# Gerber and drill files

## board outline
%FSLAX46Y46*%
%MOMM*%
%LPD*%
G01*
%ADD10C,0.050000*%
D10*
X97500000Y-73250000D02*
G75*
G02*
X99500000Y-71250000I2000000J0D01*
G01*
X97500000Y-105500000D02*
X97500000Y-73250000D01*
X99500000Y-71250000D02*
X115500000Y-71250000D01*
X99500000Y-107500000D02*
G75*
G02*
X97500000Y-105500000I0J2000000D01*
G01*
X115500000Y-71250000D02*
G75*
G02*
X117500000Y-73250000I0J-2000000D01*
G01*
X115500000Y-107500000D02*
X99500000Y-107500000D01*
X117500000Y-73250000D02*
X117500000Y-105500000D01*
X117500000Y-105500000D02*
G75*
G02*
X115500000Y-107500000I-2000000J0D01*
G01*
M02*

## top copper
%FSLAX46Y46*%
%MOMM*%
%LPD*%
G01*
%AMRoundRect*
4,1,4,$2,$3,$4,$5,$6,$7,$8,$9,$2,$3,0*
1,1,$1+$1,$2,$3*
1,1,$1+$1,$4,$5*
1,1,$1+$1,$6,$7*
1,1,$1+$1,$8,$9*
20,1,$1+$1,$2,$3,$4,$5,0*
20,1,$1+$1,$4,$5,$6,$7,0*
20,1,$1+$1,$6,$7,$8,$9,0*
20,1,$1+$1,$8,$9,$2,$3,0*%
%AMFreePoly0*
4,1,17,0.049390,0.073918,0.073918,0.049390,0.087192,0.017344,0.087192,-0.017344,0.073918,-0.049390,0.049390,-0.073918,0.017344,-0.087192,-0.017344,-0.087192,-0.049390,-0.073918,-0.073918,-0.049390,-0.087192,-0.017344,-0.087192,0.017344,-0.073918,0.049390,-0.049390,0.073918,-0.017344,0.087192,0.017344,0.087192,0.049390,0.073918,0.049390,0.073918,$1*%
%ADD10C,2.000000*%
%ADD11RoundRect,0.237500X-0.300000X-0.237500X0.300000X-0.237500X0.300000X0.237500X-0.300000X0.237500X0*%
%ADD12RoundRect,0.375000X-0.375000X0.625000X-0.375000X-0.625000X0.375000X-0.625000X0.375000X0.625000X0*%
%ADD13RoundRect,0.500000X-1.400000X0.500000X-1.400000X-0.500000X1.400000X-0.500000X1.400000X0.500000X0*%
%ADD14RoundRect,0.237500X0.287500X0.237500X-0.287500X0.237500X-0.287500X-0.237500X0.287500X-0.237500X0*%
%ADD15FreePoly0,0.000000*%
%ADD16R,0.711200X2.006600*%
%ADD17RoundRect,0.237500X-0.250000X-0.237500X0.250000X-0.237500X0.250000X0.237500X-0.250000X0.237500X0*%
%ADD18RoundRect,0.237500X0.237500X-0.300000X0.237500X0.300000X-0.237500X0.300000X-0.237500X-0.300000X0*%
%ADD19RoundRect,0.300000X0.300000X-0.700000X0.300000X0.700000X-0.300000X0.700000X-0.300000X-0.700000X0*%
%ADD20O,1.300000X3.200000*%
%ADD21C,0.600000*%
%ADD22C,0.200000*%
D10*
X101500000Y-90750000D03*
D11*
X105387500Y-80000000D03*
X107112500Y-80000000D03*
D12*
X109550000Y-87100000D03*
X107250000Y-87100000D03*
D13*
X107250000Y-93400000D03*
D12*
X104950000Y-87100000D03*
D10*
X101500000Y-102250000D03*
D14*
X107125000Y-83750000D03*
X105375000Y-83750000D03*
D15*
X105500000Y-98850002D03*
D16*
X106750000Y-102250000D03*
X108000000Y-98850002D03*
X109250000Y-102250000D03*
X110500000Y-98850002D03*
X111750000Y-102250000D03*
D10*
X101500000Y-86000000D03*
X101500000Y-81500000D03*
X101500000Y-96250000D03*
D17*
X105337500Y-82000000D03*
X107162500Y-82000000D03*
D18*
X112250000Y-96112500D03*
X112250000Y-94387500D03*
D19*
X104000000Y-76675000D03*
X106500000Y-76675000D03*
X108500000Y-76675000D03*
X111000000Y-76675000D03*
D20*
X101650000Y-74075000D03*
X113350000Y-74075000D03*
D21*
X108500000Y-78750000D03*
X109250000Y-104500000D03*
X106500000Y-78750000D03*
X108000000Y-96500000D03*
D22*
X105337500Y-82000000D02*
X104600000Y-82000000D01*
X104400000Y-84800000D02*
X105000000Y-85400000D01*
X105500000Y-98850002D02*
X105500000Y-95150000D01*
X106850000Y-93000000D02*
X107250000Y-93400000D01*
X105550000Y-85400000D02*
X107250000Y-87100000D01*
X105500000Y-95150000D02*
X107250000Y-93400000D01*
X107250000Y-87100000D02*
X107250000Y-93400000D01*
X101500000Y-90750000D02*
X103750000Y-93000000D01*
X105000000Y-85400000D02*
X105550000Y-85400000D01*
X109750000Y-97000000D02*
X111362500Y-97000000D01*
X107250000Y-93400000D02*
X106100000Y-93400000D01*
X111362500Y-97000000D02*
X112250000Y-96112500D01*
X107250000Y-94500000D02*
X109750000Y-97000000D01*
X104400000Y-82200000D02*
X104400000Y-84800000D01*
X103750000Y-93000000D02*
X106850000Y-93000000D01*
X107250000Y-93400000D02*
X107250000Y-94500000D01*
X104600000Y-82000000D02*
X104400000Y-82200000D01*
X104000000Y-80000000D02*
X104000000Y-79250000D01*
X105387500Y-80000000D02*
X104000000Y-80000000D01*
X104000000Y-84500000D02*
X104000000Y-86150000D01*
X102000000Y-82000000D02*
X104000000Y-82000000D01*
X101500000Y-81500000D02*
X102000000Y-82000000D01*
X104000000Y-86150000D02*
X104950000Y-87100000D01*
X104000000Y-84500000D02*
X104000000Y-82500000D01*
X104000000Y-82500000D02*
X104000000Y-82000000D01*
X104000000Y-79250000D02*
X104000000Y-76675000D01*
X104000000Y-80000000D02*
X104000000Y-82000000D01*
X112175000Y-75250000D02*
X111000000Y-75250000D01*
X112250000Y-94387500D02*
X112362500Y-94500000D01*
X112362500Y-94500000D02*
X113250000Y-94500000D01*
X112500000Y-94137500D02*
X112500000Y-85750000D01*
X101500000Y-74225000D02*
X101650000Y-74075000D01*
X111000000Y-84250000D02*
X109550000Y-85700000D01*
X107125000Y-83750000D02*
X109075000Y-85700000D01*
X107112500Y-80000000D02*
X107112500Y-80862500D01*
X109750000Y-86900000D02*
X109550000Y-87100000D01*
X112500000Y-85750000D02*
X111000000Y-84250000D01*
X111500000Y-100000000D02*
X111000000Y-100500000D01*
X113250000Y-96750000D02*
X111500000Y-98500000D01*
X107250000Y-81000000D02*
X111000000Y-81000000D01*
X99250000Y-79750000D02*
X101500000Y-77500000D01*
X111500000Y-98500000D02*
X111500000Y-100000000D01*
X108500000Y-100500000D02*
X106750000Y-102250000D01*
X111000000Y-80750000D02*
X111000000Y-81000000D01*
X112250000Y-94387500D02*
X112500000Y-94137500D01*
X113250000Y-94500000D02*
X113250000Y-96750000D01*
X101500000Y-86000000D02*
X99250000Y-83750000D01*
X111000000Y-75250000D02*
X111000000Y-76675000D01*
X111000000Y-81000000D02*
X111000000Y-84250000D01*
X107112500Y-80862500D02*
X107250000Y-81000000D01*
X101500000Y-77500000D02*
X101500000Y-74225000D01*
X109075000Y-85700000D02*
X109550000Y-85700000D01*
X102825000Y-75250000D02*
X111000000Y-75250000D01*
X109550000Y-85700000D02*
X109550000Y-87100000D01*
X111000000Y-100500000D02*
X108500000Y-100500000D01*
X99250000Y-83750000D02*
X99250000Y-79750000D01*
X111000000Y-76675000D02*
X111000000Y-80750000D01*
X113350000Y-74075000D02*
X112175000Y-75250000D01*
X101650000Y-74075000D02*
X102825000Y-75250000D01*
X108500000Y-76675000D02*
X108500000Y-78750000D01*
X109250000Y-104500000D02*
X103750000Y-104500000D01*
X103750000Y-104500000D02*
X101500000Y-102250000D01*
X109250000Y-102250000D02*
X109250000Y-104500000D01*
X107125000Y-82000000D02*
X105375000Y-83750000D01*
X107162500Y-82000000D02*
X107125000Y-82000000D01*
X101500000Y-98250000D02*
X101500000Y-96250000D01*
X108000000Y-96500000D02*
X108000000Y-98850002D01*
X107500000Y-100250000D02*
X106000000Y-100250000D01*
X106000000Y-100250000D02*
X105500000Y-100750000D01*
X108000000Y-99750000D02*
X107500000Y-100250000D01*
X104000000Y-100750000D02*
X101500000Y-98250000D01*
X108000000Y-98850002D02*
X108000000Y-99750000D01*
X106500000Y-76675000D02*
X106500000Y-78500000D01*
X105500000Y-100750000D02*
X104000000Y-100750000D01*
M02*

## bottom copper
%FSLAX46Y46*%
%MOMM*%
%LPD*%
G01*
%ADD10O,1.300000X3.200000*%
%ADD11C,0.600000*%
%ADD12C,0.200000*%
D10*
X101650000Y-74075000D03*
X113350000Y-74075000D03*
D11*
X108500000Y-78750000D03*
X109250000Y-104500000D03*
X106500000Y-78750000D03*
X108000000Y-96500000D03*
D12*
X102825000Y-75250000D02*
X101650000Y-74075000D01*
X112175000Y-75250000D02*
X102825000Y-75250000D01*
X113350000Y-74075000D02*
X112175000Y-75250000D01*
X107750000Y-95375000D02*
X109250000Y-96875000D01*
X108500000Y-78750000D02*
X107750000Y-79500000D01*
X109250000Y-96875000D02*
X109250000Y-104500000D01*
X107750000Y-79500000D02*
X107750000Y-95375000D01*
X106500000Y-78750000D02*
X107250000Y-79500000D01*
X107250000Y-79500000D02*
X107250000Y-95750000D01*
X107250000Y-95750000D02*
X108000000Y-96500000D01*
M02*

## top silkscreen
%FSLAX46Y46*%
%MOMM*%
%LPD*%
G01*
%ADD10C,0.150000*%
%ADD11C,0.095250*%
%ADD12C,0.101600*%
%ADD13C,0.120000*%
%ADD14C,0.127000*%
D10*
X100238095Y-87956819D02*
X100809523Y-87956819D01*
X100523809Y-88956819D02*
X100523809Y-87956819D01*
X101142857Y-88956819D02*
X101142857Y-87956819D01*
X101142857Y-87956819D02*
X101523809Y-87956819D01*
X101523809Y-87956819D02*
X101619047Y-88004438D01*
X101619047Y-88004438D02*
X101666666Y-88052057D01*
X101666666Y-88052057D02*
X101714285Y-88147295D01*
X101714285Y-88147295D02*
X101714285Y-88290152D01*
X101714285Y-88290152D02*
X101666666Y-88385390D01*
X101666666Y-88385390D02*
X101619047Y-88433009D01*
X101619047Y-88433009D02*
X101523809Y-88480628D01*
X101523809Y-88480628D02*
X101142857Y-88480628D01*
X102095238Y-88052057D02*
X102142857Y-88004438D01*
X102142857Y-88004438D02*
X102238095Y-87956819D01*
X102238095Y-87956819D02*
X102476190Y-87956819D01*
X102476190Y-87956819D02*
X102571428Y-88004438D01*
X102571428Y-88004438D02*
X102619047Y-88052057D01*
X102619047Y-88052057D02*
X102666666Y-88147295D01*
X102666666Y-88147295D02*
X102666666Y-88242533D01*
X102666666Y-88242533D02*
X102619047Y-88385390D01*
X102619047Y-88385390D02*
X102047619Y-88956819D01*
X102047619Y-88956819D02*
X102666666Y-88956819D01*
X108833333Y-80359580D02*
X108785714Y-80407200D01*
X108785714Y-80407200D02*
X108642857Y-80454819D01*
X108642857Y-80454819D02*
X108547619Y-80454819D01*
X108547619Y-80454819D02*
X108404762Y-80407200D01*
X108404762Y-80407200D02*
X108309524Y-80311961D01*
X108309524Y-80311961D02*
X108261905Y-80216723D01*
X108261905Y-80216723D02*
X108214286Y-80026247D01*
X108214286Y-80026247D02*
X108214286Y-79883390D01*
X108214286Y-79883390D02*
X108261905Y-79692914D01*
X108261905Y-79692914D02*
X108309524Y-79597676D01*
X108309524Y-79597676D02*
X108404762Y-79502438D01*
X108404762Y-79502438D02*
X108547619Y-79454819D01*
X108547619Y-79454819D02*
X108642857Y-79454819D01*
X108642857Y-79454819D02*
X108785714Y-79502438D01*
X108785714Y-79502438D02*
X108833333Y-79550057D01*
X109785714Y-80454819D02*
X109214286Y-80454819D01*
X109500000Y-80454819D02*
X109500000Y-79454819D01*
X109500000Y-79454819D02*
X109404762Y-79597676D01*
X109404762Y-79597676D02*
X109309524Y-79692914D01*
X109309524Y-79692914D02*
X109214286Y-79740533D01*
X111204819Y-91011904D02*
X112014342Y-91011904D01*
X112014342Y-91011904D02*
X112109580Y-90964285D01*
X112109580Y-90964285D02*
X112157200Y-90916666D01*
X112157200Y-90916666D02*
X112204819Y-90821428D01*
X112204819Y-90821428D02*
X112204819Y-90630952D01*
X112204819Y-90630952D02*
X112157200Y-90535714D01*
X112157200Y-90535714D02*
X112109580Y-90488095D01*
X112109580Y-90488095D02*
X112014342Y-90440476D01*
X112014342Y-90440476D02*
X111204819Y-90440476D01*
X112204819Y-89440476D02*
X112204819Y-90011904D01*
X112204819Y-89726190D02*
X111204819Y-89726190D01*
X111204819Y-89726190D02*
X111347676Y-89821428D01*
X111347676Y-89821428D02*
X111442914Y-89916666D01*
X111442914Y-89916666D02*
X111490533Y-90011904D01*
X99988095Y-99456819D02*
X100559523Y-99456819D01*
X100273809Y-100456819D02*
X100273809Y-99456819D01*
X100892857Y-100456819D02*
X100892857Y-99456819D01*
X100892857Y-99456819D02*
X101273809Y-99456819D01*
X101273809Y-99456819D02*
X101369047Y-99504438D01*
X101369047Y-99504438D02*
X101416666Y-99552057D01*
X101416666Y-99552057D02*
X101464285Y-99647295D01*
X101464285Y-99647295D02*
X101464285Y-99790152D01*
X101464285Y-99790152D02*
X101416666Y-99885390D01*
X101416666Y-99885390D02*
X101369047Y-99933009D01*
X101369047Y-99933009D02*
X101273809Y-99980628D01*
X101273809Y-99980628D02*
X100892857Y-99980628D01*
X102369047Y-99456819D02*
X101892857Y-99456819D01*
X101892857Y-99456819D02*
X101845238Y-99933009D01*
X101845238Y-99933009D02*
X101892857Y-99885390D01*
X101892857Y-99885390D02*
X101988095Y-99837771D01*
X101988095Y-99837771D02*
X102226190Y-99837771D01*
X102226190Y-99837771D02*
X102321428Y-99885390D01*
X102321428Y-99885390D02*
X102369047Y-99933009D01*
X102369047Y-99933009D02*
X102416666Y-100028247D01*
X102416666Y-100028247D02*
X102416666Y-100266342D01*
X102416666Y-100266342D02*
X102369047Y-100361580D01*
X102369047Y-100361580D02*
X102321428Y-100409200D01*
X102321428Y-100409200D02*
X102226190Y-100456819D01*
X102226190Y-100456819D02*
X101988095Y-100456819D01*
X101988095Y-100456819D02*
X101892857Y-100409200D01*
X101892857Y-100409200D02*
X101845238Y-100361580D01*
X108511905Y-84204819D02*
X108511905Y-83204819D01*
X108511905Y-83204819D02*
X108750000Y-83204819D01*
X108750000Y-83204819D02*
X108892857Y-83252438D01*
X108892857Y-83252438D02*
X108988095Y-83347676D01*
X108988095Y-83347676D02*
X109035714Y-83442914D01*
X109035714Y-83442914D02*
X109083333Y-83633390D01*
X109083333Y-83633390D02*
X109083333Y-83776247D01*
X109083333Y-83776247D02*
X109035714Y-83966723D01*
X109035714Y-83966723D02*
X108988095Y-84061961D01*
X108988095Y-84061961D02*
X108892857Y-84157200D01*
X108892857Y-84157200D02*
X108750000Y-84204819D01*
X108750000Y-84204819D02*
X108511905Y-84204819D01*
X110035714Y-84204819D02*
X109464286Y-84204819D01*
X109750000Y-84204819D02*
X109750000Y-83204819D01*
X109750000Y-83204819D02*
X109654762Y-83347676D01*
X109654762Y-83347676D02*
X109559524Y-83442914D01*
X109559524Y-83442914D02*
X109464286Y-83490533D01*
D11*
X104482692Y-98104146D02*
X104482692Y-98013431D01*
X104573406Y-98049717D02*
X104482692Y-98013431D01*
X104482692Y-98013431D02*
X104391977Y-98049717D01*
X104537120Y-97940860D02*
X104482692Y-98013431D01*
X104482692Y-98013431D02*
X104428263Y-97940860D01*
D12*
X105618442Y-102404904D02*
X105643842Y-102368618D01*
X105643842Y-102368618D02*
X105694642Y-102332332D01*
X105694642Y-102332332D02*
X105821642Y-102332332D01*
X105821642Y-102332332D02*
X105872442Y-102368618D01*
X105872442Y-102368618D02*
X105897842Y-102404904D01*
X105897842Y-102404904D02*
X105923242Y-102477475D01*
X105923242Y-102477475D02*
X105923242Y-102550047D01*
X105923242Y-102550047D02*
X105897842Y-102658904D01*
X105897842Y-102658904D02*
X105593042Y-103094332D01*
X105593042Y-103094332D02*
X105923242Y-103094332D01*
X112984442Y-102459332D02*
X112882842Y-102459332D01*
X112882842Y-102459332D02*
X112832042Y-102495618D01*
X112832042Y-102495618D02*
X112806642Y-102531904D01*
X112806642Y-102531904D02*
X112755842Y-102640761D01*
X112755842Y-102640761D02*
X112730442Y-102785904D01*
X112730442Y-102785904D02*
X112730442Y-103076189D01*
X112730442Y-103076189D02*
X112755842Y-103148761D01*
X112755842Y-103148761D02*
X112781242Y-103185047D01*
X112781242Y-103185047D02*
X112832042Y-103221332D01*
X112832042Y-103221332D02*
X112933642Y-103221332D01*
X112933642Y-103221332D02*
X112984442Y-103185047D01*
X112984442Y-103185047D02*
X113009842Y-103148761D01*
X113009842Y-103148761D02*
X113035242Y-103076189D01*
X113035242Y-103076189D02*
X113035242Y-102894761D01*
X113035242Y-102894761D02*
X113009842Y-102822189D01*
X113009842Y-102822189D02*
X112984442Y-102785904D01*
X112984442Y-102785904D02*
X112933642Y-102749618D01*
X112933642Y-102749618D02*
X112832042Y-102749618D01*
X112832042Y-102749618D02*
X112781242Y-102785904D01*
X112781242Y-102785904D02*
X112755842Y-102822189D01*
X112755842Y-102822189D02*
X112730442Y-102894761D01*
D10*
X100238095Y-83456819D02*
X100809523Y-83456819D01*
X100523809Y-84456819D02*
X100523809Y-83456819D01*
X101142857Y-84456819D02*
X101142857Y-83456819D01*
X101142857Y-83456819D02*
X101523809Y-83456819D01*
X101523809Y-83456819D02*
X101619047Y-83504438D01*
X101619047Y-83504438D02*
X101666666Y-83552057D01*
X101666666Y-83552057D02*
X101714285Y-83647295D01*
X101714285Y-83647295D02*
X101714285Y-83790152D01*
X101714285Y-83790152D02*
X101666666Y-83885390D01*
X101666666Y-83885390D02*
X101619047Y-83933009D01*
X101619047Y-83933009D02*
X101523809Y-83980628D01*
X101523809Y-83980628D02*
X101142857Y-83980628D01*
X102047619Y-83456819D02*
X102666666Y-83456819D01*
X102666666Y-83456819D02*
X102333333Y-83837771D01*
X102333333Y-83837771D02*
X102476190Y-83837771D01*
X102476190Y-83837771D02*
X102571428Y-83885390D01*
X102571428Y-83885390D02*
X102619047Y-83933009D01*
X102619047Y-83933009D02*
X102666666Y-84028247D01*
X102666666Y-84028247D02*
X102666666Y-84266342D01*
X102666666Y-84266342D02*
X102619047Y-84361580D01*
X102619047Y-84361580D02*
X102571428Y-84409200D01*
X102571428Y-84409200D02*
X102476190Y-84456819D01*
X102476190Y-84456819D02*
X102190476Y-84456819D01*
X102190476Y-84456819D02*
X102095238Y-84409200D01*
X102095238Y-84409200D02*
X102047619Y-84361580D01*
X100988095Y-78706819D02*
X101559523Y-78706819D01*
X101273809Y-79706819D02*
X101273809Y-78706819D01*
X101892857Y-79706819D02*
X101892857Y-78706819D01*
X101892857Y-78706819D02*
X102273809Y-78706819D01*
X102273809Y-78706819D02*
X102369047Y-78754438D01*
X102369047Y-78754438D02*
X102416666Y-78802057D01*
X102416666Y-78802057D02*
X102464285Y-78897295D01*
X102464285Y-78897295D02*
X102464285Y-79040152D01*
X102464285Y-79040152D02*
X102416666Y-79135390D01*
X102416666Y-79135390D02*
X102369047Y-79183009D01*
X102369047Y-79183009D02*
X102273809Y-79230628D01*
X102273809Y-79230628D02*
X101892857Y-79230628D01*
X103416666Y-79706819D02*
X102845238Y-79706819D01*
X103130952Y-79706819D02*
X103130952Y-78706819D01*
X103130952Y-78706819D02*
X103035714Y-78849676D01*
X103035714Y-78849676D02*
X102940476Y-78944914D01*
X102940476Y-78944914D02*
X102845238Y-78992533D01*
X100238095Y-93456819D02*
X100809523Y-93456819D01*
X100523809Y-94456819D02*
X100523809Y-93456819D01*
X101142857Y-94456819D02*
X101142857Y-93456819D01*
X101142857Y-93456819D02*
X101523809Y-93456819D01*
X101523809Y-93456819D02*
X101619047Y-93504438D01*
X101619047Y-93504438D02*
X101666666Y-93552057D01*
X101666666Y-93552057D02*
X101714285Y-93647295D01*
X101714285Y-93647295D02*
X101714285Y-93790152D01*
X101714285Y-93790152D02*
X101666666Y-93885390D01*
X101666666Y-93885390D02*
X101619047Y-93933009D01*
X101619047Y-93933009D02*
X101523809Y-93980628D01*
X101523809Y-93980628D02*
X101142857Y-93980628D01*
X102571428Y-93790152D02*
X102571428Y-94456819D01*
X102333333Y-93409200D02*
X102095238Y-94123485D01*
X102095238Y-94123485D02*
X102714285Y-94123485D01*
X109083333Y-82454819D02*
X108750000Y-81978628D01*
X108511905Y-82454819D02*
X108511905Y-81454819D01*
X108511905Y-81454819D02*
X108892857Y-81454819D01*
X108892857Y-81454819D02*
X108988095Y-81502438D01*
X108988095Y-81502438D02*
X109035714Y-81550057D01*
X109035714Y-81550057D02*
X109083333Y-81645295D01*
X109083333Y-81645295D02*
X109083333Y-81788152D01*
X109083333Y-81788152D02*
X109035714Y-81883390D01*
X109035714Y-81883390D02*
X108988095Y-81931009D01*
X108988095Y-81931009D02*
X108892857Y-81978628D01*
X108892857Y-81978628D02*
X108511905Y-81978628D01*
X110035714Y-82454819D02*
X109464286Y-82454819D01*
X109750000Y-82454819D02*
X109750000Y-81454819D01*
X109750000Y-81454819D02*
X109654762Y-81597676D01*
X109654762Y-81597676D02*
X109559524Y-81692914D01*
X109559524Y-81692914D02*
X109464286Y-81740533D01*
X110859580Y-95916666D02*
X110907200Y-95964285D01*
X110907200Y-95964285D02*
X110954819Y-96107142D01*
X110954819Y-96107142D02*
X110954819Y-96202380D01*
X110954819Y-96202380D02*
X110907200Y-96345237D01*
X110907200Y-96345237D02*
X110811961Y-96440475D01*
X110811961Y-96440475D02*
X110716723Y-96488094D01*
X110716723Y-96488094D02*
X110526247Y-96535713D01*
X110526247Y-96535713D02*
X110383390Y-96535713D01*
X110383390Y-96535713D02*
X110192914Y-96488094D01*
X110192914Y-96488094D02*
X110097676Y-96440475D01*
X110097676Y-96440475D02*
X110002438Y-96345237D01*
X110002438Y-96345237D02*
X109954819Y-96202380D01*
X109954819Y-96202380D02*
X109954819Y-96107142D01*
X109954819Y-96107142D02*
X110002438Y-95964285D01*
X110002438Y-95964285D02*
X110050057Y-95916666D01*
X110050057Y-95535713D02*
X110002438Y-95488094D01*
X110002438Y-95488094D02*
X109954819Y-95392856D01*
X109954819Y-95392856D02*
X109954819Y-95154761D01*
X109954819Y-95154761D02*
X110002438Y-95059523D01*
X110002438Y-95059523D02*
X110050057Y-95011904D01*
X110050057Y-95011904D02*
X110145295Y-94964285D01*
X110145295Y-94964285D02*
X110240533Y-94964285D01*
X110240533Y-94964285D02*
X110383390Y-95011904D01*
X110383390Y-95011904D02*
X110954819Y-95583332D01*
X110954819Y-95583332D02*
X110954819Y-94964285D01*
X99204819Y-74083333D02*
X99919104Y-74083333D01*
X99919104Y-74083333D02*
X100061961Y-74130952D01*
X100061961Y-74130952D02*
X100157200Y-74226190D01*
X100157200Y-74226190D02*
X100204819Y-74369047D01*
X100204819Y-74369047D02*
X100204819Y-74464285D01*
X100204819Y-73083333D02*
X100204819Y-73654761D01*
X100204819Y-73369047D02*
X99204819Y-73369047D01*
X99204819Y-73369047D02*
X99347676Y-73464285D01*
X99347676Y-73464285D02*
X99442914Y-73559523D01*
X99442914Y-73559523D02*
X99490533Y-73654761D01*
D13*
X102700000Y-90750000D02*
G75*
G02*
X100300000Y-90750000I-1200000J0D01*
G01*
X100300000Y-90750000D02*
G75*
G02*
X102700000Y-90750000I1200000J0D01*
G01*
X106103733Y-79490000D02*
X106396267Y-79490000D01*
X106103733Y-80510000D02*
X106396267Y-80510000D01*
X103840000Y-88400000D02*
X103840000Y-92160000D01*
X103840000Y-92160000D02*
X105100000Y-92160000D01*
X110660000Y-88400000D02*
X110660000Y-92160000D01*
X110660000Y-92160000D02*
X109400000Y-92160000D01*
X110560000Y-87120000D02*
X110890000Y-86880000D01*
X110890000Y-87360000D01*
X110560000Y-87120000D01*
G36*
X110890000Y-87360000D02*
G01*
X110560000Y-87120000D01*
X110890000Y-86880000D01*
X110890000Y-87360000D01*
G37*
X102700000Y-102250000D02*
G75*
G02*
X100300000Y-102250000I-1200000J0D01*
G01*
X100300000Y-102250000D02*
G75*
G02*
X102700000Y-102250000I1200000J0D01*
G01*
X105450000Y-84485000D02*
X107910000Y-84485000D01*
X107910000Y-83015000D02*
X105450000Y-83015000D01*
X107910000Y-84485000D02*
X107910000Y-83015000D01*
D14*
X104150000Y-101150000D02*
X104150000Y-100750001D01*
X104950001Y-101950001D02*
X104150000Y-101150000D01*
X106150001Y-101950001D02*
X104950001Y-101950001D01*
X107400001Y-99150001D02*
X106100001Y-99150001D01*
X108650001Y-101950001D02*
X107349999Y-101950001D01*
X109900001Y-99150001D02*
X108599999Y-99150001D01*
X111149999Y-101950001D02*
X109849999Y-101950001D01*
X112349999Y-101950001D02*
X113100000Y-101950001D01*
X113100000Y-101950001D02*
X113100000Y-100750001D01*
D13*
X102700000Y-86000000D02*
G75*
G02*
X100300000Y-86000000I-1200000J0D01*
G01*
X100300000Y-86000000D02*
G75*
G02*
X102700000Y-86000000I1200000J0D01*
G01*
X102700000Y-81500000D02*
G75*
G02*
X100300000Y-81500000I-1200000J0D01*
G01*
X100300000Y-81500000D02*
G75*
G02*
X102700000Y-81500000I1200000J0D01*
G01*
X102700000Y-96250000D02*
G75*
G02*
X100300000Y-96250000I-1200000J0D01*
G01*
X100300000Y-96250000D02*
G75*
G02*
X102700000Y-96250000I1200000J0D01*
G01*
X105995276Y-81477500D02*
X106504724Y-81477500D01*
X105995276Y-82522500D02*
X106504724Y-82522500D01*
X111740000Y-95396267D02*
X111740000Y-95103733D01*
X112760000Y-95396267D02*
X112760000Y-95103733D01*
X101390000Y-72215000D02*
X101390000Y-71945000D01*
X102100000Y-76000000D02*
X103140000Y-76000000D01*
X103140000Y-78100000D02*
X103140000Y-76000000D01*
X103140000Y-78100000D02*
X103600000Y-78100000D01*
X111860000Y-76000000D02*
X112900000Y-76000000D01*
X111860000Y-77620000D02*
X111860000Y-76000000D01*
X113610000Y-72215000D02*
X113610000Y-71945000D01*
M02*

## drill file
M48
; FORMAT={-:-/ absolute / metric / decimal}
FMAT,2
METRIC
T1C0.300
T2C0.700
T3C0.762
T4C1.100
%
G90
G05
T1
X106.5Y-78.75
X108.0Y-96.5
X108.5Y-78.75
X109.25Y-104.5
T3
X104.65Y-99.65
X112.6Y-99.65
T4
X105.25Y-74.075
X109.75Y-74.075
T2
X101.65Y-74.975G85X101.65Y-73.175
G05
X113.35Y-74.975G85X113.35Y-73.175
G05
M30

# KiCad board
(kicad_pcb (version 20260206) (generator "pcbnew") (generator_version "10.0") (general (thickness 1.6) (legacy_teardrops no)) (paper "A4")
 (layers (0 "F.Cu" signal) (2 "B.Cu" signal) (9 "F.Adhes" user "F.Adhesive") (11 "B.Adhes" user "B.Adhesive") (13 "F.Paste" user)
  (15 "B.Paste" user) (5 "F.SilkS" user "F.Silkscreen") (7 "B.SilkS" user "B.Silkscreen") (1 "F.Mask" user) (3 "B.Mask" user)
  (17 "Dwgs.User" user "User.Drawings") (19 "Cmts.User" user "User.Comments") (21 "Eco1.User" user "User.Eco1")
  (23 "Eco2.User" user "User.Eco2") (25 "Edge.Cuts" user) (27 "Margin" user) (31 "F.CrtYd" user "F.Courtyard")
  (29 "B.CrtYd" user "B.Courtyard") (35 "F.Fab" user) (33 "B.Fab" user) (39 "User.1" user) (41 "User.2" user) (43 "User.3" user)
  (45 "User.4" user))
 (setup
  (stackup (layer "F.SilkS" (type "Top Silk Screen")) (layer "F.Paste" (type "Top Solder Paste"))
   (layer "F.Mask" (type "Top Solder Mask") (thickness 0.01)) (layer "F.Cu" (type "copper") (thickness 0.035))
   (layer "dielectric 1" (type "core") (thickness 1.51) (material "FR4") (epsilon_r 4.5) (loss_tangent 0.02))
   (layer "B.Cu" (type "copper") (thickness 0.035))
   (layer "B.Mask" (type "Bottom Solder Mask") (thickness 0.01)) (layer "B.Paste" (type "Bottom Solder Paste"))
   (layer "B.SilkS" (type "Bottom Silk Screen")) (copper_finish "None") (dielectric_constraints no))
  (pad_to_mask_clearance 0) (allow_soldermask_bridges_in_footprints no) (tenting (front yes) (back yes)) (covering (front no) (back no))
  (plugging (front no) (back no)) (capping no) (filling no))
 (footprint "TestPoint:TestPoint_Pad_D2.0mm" (layer "F.Cu") (at 101.5 90.75)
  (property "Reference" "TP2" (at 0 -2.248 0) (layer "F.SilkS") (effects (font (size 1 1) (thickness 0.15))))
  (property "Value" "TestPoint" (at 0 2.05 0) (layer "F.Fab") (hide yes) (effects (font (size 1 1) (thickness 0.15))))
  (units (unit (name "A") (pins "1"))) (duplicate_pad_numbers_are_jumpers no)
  (fp_circle (center 0 0) (end 0 1.2) (stroke (width 0.12) (type solid)) (fill no) (layer "F.SilkS"))
  (pad "1" smd circle (at 0 0) (size 2 2) (layers "F.Cu" "F.Mask") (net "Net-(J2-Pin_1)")))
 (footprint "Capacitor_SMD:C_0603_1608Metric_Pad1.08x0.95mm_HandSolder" (layer "F.Cu") (at 106.25 80)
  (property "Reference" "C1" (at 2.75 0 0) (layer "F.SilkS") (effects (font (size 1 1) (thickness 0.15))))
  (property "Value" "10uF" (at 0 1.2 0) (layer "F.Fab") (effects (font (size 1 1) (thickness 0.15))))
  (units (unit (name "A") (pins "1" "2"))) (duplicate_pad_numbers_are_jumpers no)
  (fp_line (start -0.146267 -0.51) (end 0.146267 -0.51) (stroke (width 0.12) (type solid)) (layer "F.SilkS"))
  (fp_line (start -0.146267 0.51) (end 0.146267 0.51) (stroke (width 0.12) (type solid)) (layer "F.SilkS"))
  (pad "1" smd roundrect (at -0.8625 0) (size 1.075 0.95) (layers "F.Cu" "F.Mask" "F.Paste") (roundrect_rratio 0.25) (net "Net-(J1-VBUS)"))
  (pad "2" smd roundrect (at 0.8625 0) (size 1.075 0.95) (layers "F.Cu" "F.Mask" "F.Paste") (roundrect_rratio 0.25) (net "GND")))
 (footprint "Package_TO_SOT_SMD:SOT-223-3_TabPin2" (layer "F.Cu") (at 107.25 90.25 -90)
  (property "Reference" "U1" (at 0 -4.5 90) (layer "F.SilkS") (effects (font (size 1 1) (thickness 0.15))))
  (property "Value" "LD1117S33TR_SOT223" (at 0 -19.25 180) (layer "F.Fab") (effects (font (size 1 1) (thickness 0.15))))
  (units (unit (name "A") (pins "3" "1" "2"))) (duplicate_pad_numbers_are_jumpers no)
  (fp_line (start -1.85 3.41) (end 1.91 3.41) (stroke (width 0.12) (type solid)) (layer "F.SilkS"))
  (fp_line (start 1.91 3.41) (end 1.91 2.15) (stroke (width 0.12) (type solid)) (layer "F.SilkS"))
  (fp_line (start -1.85 -3.41) (end 1.91 -3.41) (stroke (width 0.12) (type solid)) (layer "F.SilkS"))
  (fp_line (start 1.91 -3.41) (end 1.91 -2.15) (stroke (width 0.12) (type solid)) (layer "F.SilkS"))
  (fp_poly
   (pts (xy -3.13 -3.31) (xy -3.37 -3.64) (xy -2.89 -3.64) (xy -3.13 -3.31)) (stroke (width 0.12) (type solid)) (fill yes) (layer "F.SilkS"))
  (pad "1" smd roundrect (at -3.15 -2.3 270) (size 2 1.5) (layers "F.Cu" "F.Mask" "F.Paste") (roundrect_rratio 0.25) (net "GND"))
  (pad "2" smd roundrect (at -3.15 0 270) (size 2 1.5) (layers "F.Cu" "F.Mask" "F.Paste") (roundrect_rratio 0.25) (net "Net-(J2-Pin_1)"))
  (pad "2" smd roundrect (at 3.15 0 270) (size 2 3.8) (layers "F.Cu" "F.Mask" "F.Paste") (roundrect_rratio 0.25) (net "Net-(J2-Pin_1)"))
  (pad "3" smd roundrect (at -3.15 2.3 270) (size 2 1.5) (layers "F.Cu" "F.Mask" "F.Paste") (roundrect_rratio 0.25) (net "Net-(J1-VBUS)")))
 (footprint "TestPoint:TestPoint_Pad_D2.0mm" (layer "F.Cu") (at 101.5 102.25)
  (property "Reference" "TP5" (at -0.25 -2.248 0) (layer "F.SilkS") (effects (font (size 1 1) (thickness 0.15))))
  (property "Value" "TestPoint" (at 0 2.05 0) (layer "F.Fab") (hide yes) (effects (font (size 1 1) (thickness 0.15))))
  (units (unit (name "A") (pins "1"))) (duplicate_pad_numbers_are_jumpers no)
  (fp_circle (center 0 0) (end 0 1.2) (stroke (width 0.12) (type solid)) (fill no) (layer "F.SilkS"))
  (pad "1" smd circle (at 0 0) (size 2 2) (layers "F.Cu" "F.Mask") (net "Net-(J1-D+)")))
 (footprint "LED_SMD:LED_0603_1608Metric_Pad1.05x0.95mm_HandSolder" (layer "F.Cu") (at 106.25 83.75 180)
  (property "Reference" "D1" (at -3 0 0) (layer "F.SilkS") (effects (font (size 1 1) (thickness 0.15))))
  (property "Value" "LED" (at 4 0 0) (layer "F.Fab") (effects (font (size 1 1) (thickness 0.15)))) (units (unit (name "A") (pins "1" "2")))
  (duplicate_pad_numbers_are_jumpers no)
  (fp_line (start 0.8 -0.735) (end -1.66 -0.735) (stroke (width 0.12) (type solid)) (layer "F.SilkS"))
  (fp_line (start -1.66 0.735) (end 0.8 0.735) (stroke (width 0.12) (type solid)) (layer "F.SilkS"))
  (fp_line (start -1.66 -0.735) (end -1.66 0.735) (stroke (width 0.12) (type solid)) (layer "F.SilkS"))
  (pad "1" smd roundrect (at -0.875 0 180) (size 1.05 0.95) (layers "F.Cu" "F.Mask" "F.Paste") (roundrect_rratio 0.25) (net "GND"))
  (pad "2" smd roundrect (at 0.875 0 180) (size 1.05 0.95) (layers "F.Cu" "F.Mask" "F.Paste") (roundrect_rratio 0.25) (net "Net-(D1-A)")))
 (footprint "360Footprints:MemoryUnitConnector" (layer "F.Cu") (at 108.625 100.550001)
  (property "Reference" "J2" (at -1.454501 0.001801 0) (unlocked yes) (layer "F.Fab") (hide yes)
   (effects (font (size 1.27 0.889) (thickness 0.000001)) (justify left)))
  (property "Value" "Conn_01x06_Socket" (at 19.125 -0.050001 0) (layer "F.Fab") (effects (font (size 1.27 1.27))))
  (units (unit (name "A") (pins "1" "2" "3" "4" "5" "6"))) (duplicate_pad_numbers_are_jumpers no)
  (fp_line (start -4.475 0.599999) (end -4.475 0.2) (stroke (width 0.127) (type default)) (layer "F.SilkS"))
  (fp_line (start -3.674999 1.4) (end -4.475 0.599999) (stroke (width 0.127) (type default)) (layer "F.SilkS"))
  (fp_line (start -2.474999 1.4) (end -3.674999 1.4) (stroke (width 0.127) (type default)) (layer "F.SilkS"))
  (fp_line (start -1.224999 -1.4) (end -2.524999 -1.4) (stroke (width 0.127) (type default)) (layer "F.SilkS"))
  (fp_line (start 0.025001 1.4) (end -1.275001 1.4) (stroke (width 0.127) (type default)) (layer "F.SilkS"))
  (fp_line (start 1.275001 -1.4) (end -0.025001 -1.4) (stroke (width 0.127) (type default)) (layer "F.SilkS"))
  (fp_line (start 2.524999 1.4) (end 1.224999 1.4) (stroke (width 0.127) (type default)) (layer "F.SilkS"))
  (fp_line (start 3.724999 1.4) (end 4.475 1.4) (stroke (width 0.127) (type default)) (layer "F.SilkS"))
  (fp_line (start 4.475 1.4) (end 4.475 0.2) (stroke (width 0.127) (type default)) (layer "F.SilkS"))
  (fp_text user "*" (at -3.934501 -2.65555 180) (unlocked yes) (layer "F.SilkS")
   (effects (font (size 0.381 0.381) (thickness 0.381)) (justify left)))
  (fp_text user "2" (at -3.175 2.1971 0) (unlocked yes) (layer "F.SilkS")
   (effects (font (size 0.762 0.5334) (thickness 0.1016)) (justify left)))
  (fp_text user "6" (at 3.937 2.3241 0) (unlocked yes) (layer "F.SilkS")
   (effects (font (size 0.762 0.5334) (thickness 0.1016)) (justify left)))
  (pad "" np_thru_hole circle (at -3.975001 -0.900001) (size 0.508 0.508) (drill 0.762) (layers "*.Cu" "*.Mask"))
  (pad "" np_thru_hole circle (at 3.975001 -0.900001) (size 0.508 0.508) (drill 0.762) (layers "*.Cu" "*.Mask"))
  (pad "1" smd custom (at -3.125 -1.699999) (size 0.1778 0.1778) (layers "F.Cu" "F.Mask" "F.Paste") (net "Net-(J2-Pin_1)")
   (options (clearance outline) (anchor circle)) (primitives))
  (pad "2" smd rect (at -1.875 1.699999) (size 0.7112 2.0066) (layers "F.Cu" "F.Mask" "F.Paste") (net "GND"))
  (pad "3" smd rect (at -0.625 -1.699999) (size 0.7112 2.0066) (layers "F.Cu" "F.Mask" "F.Paste") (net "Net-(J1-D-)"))
  (pad "4" smd rect (at 0.625 1.699999) (size 0.7112 2.0066) (layers "F.Cu" "F.Mask" "F.Paste") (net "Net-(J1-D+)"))
  (pad "5" smd rect (at 1.875 -1.699999) (size 0.7112 2.0066) (layers "F.Cu" "F.Mask" "F.Paste") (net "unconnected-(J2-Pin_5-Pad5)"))
  (pad "6" smd rect (at 3.125 1.699999) (size 0.7112 2.0066) (layers "F.Cu" "F.Mask" "F.Paste") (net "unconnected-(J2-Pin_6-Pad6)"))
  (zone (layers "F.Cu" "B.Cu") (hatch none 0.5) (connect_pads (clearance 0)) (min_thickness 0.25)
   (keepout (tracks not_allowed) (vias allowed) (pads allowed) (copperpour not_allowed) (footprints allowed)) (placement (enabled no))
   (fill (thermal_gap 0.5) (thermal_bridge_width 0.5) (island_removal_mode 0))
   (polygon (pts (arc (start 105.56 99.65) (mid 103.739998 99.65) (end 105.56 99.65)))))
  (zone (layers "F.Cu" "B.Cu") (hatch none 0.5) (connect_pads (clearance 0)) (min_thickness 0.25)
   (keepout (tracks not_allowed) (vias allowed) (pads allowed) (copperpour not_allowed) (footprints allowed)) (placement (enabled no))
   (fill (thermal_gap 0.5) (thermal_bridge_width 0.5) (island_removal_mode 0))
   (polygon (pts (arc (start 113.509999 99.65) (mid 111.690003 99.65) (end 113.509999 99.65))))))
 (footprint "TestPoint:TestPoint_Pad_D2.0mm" (layer "F.Cu") (at 101.5 86)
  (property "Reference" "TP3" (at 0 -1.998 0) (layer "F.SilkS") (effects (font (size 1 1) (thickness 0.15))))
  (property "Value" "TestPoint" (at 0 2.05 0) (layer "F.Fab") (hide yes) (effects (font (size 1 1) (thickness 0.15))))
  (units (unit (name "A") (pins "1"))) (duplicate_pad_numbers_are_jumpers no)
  (fp_circle (center 0 0) (end 0 1.2) (stroke (width 0.12) (type solid)) (fill no) (layer "F.SilkS"))
  (pad "1" smd circle (at 0 0) (size 2 2) (layers "F.Cu" "F.Mask") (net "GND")))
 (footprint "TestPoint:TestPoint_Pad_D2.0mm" (layer "F.Cu") (at 101.5 81.5)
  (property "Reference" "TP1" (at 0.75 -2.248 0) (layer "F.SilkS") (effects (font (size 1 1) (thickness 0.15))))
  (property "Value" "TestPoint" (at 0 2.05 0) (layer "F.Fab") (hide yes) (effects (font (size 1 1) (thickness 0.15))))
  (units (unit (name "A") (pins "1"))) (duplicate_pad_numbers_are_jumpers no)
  (fp_circle (center 0 0) (end 0 1.2) (stroke (width 0.12) (type solid)) (fill no) (layer "F.SilkS"))
  (pad "1" smd circle (at 0 0) (size 2 2) (layers "F.Cu" "F.Mask") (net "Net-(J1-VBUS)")))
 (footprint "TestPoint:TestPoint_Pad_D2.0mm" (layer "F.Cu") (at 101.5 96.25)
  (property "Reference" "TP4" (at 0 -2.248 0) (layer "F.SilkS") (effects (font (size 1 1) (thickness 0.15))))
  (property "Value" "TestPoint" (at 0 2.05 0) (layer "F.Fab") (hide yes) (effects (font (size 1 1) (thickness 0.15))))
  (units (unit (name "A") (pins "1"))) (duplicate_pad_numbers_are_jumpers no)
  (fp_circle (center 0 0) (end 0 1.2) (stroke (width 0.12) (type solid)) (fill no) (layer "F.SilkS"))
  (pad "1" smd circle (at 0 0) (size 2 2) (layers "F.Cu" "F.Mask") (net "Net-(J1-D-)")))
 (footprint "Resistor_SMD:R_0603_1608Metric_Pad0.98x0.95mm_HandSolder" (layer "F.Cu") (at 106.25 82)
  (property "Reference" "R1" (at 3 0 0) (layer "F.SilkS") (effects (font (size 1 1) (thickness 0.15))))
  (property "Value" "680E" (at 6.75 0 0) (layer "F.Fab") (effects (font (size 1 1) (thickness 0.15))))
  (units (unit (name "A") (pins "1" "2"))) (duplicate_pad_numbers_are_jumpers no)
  (fp_line (start -0.254724 -0.5225) (end 0.254724 -0.5225) (stroke (width 0.12) (type solid)) (layer "F.SilkS"))
  (fp_line (start -0.254724 0.5225) (end 0.254724 0.5225) (stroke (width 0.12) (type solid)) (layer "F.SilkS"))
  (pad "1" smd roundrect (at -0.9125 0) (size 0.975 0.95) (layers "F.Cu" "F.Mask" "F.Paste") (roundrect_rratio 0.25) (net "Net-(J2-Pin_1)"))
  (pad "2" smd roundrect (at 0.9125 0) (size 0.975 0.95) (layers "F.Cu" "F.Mask" "F.Paste") (roundrect_rratio 0.25) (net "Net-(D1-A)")))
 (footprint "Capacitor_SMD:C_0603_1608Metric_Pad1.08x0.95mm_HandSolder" (layer "F.Cu") (at 112.25 95.25 90)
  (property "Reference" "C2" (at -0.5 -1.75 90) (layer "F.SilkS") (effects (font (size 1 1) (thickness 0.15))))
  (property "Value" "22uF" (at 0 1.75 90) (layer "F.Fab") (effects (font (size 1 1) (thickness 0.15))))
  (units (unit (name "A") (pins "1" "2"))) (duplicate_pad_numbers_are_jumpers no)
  (fp_line (start -0.146267 -0.51) (end 0.146267 -0.51) (stroke (width 0.12) (type solid)) (layer "F.SilkS"))
  (fp_line (start -0.146267 0.51) (end 0.146267 0.51) (stroke (width 0.12) (type solid)) (layer "F.SilkS"))
  (pad "1" smd roundrect (at -0.8625 0 90) (size 1.075 0.95) (layers "F.Cu" "F.Mask" "F.Paste") (roundrect_rratio 0.25)
   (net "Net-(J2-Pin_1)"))
  (pad "2" smd roundrect (at 0.8625 0 90) (size 1.075 0.95) (layers "F.Cu" "F.Mask" "F.Paste") (roundrect_rratio 0.25) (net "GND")))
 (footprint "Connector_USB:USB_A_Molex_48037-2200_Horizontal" (layer "F.Cu") (at 107.5 65.7 90)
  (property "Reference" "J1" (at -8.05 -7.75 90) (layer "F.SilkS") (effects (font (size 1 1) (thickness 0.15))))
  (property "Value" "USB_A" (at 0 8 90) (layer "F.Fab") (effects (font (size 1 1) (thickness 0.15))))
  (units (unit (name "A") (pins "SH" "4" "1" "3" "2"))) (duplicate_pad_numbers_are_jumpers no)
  (fp_line (start -6.515 -6.11) (end -6.245 -6.11) (stroke (width 0.12) (type solid)) (layer "F.SilkS"))
  (fp_line (start -10.3 -5.4) (end -10.3 -4.36) (stroke (width 0.12) (type default)) (layer "F.SilkS"))
  (fp_line (start -12.4 -4.36) (end -10.3 -4.36) (stroke (width 0.12) (type default)) (layer "F.SilkS"))
  (fp_line (start -12.4 -4.36) (end -12.4 -3.9) (stroke (width 0.12) (type default)) (layer "F.SilkS"))
  (fp_line (start -10.3 4.36) (end -10.3 5.4) (stroke (width 0.12) (type default)) (layer "F.SilkS"))
  (fp_line (start -11.92 4.36) (end -10.3 4.36) (stroke (width 0.12) (type default)) (layer "F.SilkS"))
  (fp_line (start -6.515 6.11) (end -6.245 6.11) (stroke (width 0.12) (type solid)) (layer "F.SilkS"))
  (pad "" np_thru_hole circle (at -8.375 -2.25 90) (size 1.1 1.1) (drill 1.1) (layers "*.Mask"))
  (pad "" np_thru_hole circle (at -8.375 2.25 90) (size 1.1 1.1) (drill 1.1) (layers "*.Mask"))
  (pad "1" smd roundrect (at -10.975 -3.5 90) (size 2 1.2) (layers "F.Cu" "F.Mask" "F.Paste") (roundrect_rratio 0.25) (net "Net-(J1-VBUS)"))
  (pad "2" smd roundrect (at -10.975 -1 90) (size 2 1.2) (layers "F.Cu" "F.Mask" "F.Paste") (roundrect_rratio 0.25) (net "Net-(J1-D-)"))
  (pad "3" smd roundrect (at -10.975 1 90) (size 2 1.2) (layers "F.Cu" "F.Mask" "F.Paste") (roundrect_rratio 0.25) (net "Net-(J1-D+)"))
  (pad "4" smd roundrect (at -10.975 3.5 90) (size 2 1.2) (layers "F.Cu" "F.Mask" "F.Paste") (roundrect_rratio 0.25) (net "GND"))
  (pad "SH" thru_hole oval (at -8.375 -5.85 90) (size 3.2 1.3) (drill oval 2.5 0.7) (layers "*.Cu" "*.Mask") (remove_unused_layers no)
   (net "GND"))
  (pad "SH" thru_hole oval (at -8.375 5.85 90) (size 3.2 1.3) (drill oval 2.5 0.7) (layers "*.Cu" "*.Mask") (remove_unused_layers no)
   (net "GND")))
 (gr_arc (start 97.5 73.25) (mid 98.085786 71.835786) (end 99.5 71.25) (stroke (width 0.05) (type default)) (layer "Edge.Cuts"))
 (gr_line (start 97.5 105.5) (end 97.5 73.25) (stroke (width 0.05) (type default)) (layer "Edge.Cuts"))
 (gr_line (start 99.5 71.25) (end 115.5 71.25) (stroke (width 0.05) (type default)) (layer "Edge.Cuts"))
 (gr_arc (start 99.5 107.5) (mid 98.085786 106.914214) (end 97.5 105.5) (stroke (width 0.05) (type default)) (layer "Edge.Cuts"))
 (gr_arc (start 115.5 71.25) (mid 116.914214 71.835786) (end 117.5 73.25) (stroke (width 0.05) (type default)) (layer "Edge.Cuts"))
 (gr_line (start 115.5 107.5) (end 99.5 107.5) (stroke (width 0.05) (type default)) (layer "Edge.Cuts"))
 (gr_line (start 117.5 73.25) (end 117.5 105.5) (stroke (width 0.05) (type default)) (layer "Edge.Cuts"))
 (gr_arc (start 117.5 105.5) (mid 116.914214 106.914214) (end 115.5 107.5) (stroke (width 0.05) (type default)) (layer "Edge.Cuts"))
 (segment (start 105.3375 82) (end 104.6 82) (width 0.2) (layer "F.Cu") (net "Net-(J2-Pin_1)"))
 (segment (start 104.4 84.8) (end 105 85.4) (width 0.2) (layer "F.Cu") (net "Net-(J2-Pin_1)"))
 (segment (start 105.5 98.850002) (end 105.5 95.15) (width 0.2) (layer "F.Cu") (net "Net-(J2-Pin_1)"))
 (segment (start 106.85 93) (end 107.25 93.4) (width 0.2) (layer "F.Cu") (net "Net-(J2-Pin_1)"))
 (segment (start 105.55 85.4) (end 107.25 87.1) (width 0.2) (layer "F.Cu") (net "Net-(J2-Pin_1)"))
 (segment (start 105.5 95.15) (end 107.25 93.4) (width 0.2) (layer "F.Cu") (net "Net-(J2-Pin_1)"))
 (segment (start 107.25 87.1) (end 107.25 93.4) (width 0.2) (layer "F.Cu") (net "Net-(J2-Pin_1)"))
 (segment (start 101.5 90.75) (end 103.75 93) (width 0.2) (layer "F.Cu") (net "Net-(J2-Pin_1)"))
 (segment (start 105 85.4) (end 105.55 85.4) (width 0.2) (layer "F.Cu") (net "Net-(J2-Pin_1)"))
 (segment (start 109.75 97) (end 111.3625 97) (width 0.2) (layer "F.Cu") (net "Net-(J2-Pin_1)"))
 (segment (start 107.25 93.4) (end 106.1 93.4) (width 0.2) (layer "F.Cu") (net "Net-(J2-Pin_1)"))
 (segment (start 111.3625 97) (end 112.25 96.1125) (width 0.2) (layer "F.Cu") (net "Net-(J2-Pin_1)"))
 (segment (start 107.25 94.5) (end 109.75 97) (width 0.2) (layer "F.Cu") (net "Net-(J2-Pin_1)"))
 (segment (start 104.4 82.2) (end 104.4 84.8) (width 0.2) (layer "F.Cu") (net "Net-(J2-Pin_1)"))
 (segment (start 103.75 93) (end 106.85 93) (width 0.2) (layer "F.Cu") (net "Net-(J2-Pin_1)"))
 (segment (start 107.25 93.4) (end 107.25 94.5) (width 0.2) (layer "F.Cu") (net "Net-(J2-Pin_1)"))
 (segment (start 104.6 82) (end 104.4 82.2) (width 0.2) (layer "F.Cu") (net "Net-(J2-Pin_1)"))
 (segment (start 104 80) (end 104 79.25) (width 0.2) (layer "F.Cu") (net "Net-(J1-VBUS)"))
 (segment (start 105.3875 80) (end 104 80) (width 0.2) (layer "F.Cu") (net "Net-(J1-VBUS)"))
 (segment (start 104 84.5) (end 104 86.15) (width 0.2) (layer "F.Cu") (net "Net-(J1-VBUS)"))
 (segment (start 102 82) (end 104 82) (width 0.2) (layer "F.Cu") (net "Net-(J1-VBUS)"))
 (segment (start 101.5 81.5) (end 102 82) (width 0.2) (layer "F.Cu") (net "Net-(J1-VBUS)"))
 (segment (start 104 86.15) (end 104.95 87.1) (width 0.2) (layer "F.Cu") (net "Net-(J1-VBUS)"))
 (segment (start 104 84.5) (end 104 82.5) (width 0.2) (layer "F.Cu") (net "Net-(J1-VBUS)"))
 (segment (start 104 82.5) (end 104 82) (width 0.2) (layer "F.Cu") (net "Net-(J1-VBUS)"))
 (segment (start 104 79.25) (end 104 76.675) (width 0.2) (layer "F.Cu") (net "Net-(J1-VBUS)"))
 (segment (start 104 80) (end 104 82) (width 0.2) (layer "F.Cu") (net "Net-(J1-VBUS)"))
 (segment (start 112.175 75.25) (end 111 75.25) (width 0.2) (layer "F.Cu") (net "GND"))
 (segment (start 112.25 94.3875) (end 112.3625 94.5) (width 0.2) (layer "F.Cu") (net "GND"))
 (segment (start 112.3625 94.5) (end 113.25 94.5) (width 0.2) (layer "F.Cu") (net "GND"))
 (segment (start 112.5 94.1375) (end 112.5 85.75) (width 0.2) (layer "F.Cu") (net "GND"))
 (segment (start 101.5 74.225) (end 101.65 74.075) (width 0.2) (layer "F.Cu") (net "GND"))
 (segment (start 111 84.25) (end 109.55 85.7) (width 0.2) (layer "F.Cu") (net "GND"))
 (segment (start 107.125 83.75) (end 109.075 85.7) (width 0.2) (layer "F.Cu") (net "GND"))
 (segment (start 107.1125 80) (end 107.1125 80.8625) (width 0.2) (layer "F.Cu") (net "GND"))
 (segment (start 109.75 86.9) (end 109.55 87.1) (width 0.2) (layer "F.Cu") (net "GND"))
 (segment (start 112.5 85.75) (end 111 84.25) (width 0.2) (layer "F.Cu") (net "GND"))
 (segment (start 111.5 100) (end 111 100.5) (width 0.2) (layer "F.Cu") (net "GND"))
 (segment (start 113.25 96.75) (end 111.5 98.5) (width 0.2) (layer "F.Cu") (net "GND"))
 (segment (start 107.25 81) (end 111 81) (width 0.2) (layer "F.Cu") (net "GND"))
 (segment (start 99.25 79.75) (end 101.5 77.5) (width 0.2) (layer "F.Cu") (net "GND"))
 (segment (start 111.5 98.5) (end 111.5 100) (width 0.2) (layer "F.Cu") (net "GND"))
 (segment (start 108.5 100.5) (end 106.75 102.25) (width 0.2) (layer "F.Cu") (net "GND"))
 (segment (start 111 80.75) (end 111 81) (width 0.2) (layer "F.Cu") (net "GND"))
 (segment (start 112.25 94.3875) (end 112.5 94.1375) (width 0.2) (layer "F.Cu") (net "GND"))
 (segment (start 113.25 94.5) (end 113.25 96.75) (width 0.2) (layer "F.Cu") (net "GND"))
 (segment (start 101.5 86) (end 99.25 83.75) (width 0.2) (layer "F.Cu") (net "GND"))
 (segment (start 111 75.25) (end 111 76.675) (width 0.2) (layer "F.Cu") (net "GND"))
 (segment (start 111 81) (end 111 84.25) (width 0.2) (layer "F.Cu") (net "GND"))
 (segment (start 107.1125 80.8625) (end 107.25 81) (width 0.2) (layer "F.Cu") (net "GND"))
 (segment (start 101.5 77.5) (end 101.5 74.225) (width 0.2) (layer "F.Cu") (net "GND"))
 (segment (start 109.075 85.7) (end 109.55 85.7) (width 0.2) (layer "F.Cu") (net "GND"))
 (segment (start 102.825 75.25) (end 111 75.25) (width 0.2) (layer "F.Cu") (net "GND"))
 (segment (start 109.55 85.7) (end 109.55 87.1) (width 0.2) (layer "F.Cu") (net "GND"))
 (segment (start 111 100.5) (end 108.5 100.5) (width 0.2) (layer "F.Cu") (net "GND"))
 (segment (start 99.25 83.75) (end 99.25 79.75) (width 0.2) (layer "F.Cu") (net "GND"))
 (segment (start 111 76.675) (end 111 80.75) (width 0.2) (layer "F.Cu") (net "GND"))
 (segment (start 113.35 74.075) (end 112.175 75.25) (width 0.2) (layer "F.Cu") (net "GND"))
 (segment (start 101.65 74.075) (end 102.825 75.25) (width 0.2) (layer "F.Cu") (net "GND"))
 (segment (start 102.825 75.25) (end 101.65 74.075) (width 0.2) (layer "B.Cu") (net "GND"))
 (segment (start 112.175 75.25) (end 102.825 75.25) (width 0.2) (layer "B.Cu") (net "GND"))
 (segment (start 113.35 74.075) (end 112.175 75.25) (width 0.2) (layer "B.Cu") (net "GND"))
 (segment (start 108.5 76.675) (end 108.5 78.75) (width 0.2) (layer "F.Cu") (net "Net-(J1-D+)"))
 (segment (start 109.25 104.5) (end 103.75 104.5) (width 0.2) (layer "F.Cu") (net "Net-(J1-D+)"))
 (segment (start 103.75 104.5) (end 101.5 102.25) (width 0.2) (layer "F.Cu") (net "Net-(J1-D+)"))
 (segment (start 109.25 102.25) (end 109.25 104.5) (width 0.2) (layer "F.Cu") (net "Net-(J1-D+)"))
 (via (at 108.5 78.75) (size 0.6) (drill 0.3) (layers "F.Cu" "B.Cu") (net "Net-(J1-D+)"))
 (via (at 109.25 104.5) (size 0.6) (drill 0.3) (layers "F.Cu" "B.Cu") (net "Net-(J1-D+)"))
 (segment (start 107.75 95.375) (end 109.25 96.875) (width 0.2) (layer "B.Cu") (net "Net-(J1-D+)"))
 (segment (start 108.5 78.75) (end 107.75 79.5) (width 0.2) (layer "B.Cu") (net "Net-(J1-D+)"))
 (segment (start 109.25 96.875) (end 109.25 104.5) (width 0.2) (layer "B.Cu") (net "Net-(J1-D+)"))
 (segment (start 107.75 79.5) (end 107.75 95.375) (width 0.2) (layer "B.Cu") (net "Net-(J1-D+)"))
 (segment (start 107.125 82) (end 105.375 83.75) (width 0.2) (layer "F.Cu") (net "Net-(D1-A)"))
 (segment (start 107.1625 82) (end 107.125 82) (width 0.2) (layer "F.Cu") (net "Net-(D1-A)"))
 (segment (start 101.5 98.25) (end 101.5 96.25) (width 0.2) (layer "F.Cu") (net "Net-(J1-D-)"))
 (segment (start 108 96.5) (end 108 98.850002) (width 0.2) (layer "F.Cu") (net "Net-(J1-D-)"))
 (segment (start 107.5 100.25) (end 106 100.25) (width 0.2) (layer "F.Cu") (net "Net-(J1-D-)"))
 (segment (start 106 100.25) (end 105.5 100.75) (width 0.2) (layer "F.Cu") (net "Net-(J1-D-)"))
 (segment (start 108 99.75) (end 107.5 100.25) (width 0.2) (layer "F.Cu") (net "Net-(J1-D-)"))
 (segment (start 104 100.75) (end 101.5 98.25) (width 0.2) (layer "F.Cu") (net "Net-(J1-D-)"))
 (segment (start 108 98.850002) (end 108 99.75) (width 0.2) (layer "F.Cu") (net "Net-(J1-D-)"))
 (segment (start 106.5 76.675) (end 106.5 78.5) (width 0.2) (layer "F.Cu") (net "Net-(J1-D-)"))
 (segment (start 105.5 100.75) (end 104 100.75) (width 0.2) (layer "F.Cu") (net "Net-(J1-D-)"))
 (via (at 106.5 78.75) (size 0.6) (drill 0.3) (layers "F.Cu" "B.Cu") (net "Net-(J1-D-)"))
 (via (at 108 96.5) (size 0.6) (drill 0.3) (layers "F.Cu" "B.Cu") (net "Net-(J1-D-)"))
 (segment (start 106.5 78.75) (end 107.25 79.5) (width 0.2) (layer "B.Cu") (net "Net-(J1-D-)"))
 (segment (start 107.25 79.5) (end 107.25 95.75) (width 0.2) (layer "B.Cu") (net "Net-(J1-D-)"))
 (segment (start 107.25 95.75) (end 108 96.5) (width 0.2) (layer "B.Cu") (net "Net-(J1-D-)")))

